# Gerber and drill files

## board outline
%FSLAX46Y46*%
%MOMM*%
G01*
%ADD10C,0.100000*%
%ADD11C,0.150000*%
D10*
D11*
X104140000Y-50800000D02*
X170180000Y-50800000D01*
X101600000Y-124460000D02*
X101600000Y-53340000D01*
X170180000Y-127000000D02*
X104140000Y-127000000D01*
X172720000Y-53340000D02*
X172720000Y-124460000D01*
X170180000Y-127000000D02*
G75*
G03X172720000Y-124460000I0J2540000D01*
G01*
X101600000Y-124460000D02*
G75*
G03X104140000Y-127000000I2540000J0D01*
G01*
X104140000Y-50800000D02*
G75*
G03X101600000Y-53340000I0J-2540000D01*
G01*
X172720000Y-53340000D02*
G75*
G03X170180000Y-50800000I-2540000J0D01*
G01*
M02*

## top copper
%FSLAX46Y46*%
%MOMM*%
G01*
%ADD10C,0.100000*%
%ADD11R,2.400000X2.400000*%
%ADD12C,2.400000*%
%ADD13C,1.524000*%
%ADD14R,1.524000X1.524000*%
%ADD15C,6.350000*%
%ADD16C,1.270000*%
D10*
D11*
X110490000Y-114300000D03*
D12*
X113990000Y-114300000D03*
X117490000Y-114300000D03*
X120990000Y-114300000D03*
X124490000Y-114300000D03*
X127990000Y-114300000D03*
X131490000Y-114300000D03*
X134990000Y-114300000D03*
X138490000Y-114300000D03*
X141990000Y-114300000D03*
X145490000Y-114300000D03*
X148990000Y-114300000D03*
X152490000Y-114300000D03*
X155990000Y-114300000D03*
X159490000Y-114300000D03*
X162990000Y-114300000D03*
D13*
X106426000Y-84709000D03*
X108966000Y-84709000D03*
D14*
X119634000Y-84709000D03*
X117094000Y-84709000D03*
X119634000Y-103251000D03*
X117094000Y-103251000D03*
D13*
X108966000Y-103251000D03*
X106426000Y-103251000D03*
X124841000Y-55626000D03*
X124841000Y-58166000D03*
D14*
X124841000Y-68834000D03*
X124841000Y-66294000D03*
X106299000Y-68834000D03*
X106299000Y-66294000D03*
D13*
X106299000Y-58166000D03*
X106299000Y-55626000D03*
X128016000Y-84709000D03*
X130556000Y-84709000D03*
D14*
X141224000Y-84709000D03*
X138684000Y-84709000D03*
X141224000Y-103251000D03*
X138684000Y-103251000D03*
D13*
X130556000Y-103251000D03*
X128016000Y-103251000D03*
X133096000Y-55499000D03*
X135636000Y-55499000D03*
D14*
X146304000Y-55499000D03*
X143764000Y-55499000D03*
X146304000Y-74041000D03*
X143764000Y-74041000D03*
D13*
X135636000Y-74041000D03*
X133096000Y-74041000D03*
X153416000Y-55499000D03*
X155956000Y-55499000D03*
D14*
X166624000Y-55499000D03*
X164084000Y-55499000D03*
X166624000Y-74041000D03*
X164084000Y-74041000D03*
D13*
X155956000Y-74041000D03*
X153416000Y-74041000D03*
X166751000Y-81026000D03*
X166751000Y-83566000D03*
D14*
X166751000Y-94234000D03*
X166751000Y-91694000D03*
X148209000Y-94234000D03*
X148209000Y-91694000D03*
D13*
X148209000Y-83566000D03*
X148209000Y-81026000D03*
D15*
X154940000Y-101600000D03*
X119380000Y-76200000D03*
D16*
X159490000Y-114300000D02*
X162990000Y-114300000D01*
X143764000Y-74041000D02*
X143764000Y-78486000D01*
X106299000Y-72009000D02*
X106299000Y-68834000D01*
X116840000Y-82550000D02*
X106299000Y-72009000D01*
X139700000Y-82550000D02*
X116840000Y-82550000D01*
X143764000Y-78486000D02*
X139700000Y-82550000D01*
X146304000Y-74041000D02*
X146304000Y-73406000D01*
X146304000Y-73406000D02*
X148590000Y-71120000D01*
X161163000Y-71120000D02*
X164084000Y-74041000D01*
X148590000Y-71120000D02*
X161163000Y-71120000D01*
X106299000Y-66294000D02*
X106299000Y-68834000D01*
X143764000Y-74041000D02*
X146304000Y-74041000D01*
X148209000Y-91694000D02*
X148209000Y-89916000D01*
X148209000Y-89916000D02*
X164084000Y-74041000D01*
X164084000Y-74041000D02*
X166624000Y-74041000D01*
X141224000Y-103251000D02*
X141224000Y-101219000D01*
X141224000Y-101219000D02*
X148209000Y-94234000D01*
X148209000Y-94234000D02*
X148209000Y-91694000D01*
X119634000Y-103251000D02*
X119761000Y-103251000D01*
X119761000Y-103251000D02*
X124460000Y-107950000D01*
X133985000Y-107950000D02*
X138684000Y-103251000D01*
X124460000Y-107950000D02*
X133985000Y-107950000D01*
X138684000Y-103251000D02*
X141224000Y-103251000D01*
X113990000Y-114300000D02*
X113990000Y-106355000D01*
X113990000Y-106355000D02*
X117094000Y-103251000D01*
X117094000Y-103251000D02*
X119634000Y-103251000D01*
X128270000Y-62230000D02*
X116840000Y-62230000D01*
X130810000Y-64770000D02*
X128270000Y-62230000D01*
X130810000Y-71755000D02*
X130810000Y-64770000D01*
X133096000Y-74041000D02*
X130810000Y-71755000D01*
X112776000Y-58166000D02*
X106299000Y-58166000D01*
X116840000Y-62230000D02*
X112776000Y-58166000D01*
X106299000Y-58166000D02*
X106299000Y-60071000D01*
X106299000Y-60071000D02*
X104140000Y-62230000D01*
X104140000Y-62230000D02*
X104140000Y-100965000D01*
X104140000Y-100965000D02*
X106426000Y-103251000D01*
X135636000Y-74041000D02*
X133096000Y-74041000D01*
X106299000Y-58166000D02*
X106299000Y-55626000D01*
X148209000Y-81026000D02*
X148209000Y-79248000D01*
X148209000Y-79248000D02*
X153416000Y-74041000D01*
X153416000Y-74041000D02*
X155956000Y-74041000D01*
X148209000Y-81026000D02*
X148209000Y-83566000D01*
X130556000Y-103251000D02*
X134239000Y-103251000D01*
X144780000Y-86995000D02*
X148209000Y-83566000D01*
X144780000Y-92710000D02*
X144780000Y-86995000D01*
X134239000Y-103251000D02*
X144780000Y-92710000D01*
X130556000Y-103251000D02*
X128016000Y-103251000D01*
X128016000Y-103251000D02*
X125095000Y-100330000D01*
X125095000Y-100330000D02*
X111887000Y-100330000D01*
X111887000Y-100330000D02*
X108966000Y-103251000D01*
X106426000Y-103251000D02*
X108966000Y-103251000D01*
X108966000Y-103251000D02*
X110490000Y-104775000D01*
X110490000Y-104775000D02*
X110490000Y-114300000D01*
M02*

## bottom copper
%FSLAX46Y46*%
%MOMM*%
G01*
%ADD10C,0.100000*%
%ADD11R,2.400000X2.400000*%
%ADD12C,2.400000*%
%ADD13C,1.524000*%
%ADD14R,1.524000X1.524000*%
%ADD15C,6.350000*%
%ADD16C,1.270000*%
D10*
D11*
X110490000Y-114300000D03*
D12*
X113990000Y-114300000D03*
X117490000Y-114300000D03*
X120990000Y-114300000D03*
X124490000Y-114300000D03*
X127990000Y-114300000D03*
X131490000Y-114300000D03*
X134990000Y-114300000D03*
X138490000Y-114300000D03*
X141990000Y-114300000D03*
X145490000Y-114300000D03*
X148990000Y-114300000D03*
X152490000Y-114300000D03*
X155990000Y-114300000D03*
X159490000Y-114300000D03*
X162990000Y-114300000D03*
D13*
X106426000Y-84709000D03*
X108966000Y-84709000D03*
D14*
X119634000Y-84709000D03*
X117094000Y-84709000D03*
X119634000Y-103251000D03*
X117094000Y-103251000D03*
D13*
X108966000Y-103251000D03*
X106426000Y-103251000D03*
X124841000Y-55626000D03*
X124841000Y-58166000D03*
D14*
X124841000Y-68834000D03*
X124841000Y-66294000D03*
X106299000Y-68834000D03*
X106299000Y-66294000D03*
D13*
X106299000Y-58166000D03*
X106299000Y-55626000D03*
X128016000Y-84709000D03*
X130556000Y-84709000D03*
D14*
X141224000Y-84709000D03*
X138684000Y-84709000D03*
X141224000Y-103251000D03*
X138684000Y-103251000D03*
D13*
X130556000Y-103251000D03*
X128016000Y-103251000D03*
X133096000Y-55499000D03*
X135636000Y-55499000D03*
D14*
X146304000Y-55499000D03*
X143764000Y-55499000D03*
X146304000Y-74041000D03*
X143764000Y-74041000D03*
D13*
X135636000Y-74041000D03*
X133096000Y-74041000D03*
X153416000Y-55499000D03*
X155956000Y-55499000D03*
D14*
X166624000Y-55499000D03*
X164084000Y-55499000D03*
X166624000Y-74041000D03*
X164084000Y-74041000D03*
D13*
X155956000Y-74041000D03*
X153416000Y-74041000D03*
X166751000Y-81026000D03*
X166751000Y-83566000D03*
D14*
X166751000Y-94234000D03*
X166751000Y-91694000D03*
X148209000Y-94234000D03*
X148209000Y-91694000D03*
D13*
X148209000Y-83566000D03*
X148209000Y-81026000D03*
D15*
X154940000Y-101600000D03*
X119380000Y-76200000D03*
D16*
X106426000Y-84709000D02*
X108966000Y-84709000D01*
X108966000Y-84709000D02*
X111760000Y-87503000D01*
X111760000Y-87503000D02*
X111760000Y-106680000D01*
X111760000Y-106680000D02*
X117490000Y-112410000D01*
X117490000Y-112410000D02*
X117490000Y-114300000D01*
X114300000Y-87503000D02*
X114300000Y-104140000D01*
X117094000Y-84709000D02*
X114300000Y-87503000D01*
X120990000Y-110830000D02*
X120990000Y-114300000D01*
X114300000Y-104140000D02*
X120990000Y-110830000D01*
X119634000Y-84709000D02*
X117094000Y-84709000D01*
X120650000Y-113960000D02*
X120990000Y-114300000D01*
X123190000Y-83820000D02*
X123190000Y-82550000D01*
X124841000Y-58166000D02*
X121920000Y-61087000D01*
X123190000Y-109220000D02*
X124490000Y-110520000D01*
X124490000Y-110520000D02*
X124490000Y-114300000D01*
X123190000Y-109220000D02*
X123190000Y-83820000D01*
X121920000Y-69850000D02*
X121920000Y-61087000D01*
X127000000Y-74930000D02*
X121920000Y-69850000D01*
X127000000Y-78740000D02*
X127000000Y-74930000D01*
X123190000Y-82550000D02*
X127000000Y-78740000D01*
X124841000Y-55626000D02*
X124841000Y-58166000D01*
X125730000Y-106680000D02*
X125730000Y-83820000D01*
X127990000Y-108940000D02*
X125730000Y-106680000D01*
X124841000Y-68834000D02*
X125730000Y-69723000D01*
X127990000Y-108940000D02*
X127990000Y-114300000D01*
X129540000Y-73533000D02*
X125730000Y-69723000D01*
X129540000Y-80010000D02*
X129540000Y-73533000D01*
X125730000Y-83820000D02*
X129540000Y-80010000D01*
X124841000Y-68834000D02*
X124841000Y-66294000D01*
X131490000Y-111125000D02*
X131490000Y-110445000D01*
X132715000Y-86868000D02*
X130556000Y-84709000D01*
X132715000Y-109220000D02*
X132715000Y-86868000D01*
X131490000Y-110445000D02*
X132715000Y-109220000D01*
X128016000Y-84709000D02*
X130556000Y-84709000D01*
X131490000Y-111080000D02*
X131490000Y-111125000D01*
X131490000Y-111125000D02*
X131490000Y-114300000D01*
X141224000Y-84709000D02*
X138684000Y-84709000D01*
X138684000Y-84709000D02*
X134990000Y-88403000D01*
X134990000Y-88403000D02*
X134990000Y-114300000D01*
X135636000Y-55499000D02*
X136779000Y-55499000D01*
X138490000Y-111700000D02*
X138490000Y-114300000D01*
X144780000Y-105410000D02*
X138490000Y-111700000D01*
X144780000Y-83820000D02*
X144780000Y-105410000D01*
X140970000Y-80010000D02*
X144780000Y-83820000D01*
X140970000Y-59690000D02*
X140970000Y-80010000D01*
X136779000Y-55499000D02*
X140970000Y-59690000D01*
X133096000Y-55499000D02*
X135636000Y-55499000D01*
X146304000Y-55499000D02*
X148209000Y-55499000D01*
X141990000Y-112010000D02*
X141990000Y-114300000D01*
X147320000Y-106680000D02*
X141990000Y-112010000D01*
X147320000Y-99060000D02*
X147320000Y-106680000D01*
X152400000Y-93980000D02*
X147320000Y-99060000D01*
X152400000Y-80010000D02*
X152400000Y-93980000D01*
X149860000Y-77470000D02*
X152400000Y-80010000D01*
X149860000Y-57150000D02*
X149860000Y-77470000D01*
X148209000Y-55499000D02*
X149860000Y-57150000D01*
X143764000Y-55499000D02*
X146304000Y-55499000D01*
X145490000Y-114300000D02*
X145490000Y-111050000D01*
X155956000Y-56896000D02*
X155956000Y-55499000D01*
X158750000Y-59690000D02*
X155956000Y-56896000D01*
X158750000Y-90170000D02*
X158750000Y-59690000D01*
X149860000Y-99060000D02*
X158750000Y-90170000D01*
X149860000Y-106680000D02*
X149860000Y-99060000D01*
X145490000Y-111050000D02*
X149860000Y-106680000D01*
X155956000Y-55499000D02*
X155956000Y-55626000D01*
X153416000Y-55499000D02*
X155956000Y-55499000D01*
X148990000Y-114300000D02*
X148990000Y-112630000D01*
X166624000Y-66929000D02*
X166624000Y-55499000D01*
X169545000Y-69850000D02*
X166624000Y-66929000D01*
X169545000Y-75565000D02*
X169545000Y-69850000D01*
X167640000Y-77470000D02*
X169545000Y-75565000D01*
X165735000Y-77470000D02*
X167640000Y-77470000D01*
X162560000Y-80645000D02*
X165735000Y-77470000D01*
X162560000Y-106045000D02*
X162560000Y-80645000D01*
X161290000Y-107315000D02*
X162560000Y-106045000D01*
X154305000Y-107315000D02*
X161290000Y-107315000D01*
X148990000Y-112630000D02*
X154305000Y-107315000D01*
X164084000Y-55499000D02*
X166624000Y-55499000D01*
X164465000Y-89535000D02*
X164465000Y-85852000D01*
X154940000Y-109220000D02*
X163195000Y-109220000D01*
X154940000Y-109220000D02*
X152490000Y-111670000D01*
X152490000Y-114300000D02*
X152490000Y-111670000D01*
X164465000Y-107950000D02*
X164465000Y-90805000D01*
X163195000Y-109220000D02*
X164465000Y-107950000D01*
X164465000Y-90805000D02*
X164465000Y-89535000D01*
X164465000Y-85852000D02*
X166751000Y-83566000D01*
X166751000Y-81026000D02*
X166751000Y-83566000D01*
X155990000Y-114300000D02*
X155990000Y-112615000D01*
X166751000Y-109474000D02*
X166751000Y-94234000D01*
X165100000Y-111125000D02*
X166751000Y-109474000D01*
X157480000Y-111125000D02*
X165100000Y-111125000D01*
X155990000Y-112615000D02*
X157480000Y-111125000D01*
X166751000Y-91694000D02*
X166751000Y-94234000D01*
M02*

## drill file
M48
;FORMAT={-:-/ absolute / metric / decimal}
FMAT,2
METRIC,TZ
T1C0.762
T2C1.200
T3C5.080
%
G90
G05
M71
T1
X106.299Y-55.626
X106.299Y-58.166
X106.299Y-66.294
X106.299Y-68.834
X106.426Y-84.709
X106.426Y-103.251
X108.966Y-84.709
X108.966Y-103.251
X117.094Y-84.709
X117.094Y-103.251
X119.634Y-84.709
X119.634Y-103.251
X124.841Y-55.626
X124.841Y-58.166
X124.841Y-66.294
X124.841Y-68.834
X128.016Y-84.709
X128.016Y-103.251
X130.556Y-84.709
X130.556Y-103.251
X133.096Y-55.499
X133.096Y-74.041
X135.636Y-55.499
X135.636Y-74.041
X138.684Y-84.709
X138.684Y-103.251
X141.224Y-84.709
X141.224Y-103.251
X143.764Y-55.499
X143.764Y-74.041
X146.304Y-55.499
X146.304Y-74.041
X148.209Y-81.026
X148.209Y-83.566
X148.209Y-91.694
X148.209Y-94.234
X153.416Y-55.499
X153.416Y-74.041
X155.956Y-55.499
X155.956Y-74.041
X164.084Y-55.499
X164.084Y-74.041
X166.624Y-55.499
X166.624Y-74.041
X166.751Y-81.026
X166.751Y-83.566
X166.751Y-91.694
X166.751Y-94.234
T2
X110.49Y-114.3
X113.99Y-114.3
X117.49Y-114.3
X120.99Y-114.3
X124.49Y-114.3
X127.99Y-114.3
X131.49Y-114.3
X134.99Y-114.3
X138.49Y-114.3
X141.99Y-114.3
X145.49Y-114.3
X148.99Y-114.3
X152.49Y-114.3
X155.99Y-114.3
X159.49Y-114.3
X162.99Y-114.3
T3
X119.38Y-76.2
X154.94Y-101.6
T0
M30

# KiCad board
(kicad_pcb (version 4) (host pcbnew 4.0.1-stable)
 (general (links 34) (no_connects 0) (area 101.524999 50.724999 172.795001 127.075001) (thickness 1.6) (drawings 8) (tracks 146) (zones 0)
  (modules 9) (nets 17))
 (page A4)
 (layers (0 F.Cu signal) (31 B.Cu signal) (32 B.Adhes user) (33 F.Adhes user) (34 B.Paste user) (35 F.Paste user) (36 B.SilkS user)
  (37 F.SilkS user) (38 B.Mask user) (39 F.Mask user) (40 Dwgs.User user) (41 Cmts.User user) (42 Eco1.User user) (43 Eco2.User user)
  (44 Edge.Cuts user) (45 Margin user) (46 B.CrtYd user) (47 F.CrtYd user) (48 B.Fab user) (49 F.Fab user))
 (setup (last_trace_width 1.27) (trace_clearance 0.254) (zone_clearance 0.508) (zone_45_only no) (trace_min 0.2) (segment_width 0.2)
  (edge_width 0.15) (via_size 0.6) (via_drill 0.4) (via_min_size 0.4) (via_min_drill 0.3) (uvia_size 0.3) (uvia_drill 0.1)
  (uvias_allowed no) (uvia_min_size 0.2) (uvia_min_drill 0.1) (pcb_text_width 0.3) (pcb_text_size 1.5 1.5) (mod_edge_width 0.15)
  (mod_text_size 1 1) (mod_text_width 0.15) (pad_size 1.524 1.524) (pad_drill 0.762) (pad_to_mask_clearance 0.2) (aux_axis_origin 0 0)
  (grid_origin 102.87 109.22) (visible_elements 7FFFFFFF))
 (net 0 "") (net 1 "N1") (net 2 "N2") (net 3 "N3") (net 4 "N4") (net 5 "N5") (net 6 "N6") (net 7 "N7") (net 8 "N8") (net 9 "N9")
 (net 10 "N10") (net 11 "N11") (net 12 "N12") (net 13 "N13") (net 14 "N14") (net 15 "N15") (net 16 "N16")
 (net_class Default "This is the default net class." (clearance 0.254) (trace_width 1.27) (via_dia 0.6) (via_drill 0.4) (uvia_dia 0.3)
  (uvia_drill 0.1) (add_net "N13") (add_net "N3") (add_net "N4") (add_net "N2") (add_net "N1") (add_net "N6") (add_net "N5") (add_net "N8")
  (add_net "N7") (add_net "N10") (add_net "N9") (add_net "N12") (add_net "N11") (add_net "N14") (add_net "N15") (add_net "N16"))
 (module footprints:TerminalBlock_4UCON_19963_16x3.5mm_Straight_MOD (layer F.Cu) (at 110.49 114.3)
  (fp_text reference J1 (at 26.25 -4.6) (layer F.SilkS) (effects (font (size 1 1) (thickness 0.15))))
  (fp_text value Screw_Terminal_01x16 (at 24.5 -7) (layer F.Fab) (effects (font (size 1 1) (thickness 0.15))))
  (pad 1 thru_hole rect (at 0 0) (size 2.4 2.4) (drill 1.2) (layers *.Cu *.Mask))
  (pad 2 thru_hole circle (at 3.5 0) (size 2.4 2.4) (drill 1.2) (layers *.Cu *.Mask))
  (pad 3 thru_hole circle (at 7 0) (size 2.4 2.4) (drill 1.2) (layers *.Cu *.Mask))
  (pad 4 thru_hole circle (at 10.5 0) (size 2.4 2.4) (drill 1.2) (layers *.Cu *.Mask))
  (pad 5 thru_hole circle (at 14 0) (size 2.4 2.4) (drill 1.2) (layers *.Cu *.Mask))
  (pad 6 thru_hole circle (at 17.5 0) (size 2.4 2.4) (drill 1.2) (layers *.Cu *.Mask))
  (pad 7 thru_hole circle (at 21 0) (size 2.4 2.4) (drill 1.2) (layers *.Cu *.Mask))
  (pad 8 thru_hole circle (at 24.5 0) (size 2.4 2.4) (drill 1.2) (layers *.Cu *.Mask))
  (pad 9 thru_hole circle (at 28 0) (size 2.4 2.4) (drill 1.2) (layers *.Cu *.Mask))
  (pad 10 thru_hole circle (at 31.5 0) (size 2.4 2.4) (drill 1.2) (layers *.Cu *.Mask))
  (pad 11 thru_hole circle (at 35 0) (size 2.4 2.4) (drill 1.2) (layers *.Cu *.Mask))
  (pad 12 thru_hole circle (at 38.5 0) (size 2.4 2.4) (drill 1.2) (layers *.Cu *.Mask))
  (pad 13 thru_hole circle (at 42 0) (size 2.4 2.4) (drill 1.2) (layers *.Cu *.Mask))
  (pad 14 thru_hole circle (at 45.5 0) (size 2.4 2.4) (drill 1.2) (layers *.Cu *.Mask))
  (pad 15 thru_hole circle (at 49 0) (size 2.4 2.4) (drill 1.2) (layers *.Cu *.Mask))
  (pad 16 thru_hole circle (at 52.5 0) (size 2.4 2.4) (drill 1.2) (layers *.Cu *.Mask)))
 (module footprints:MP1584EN (layer F.Cu) (at 113.03 93.98 90)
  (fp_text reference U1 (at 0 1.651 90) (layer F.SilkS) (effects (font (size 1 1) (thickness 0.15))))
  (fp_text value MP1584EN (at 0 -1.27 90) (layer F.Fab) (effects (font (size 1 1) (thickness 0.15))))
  (pad 4 thru_hole circle (at 9.271 -6.604 90) (size 1.524 1.524) (drill 0.762) (layers *.Cu *.Mask) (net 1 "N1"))
  (pad 4 thru_hole circle (at 9.271 -4.064 90) (size 1.524 1.524) (drill 0.762) (layers *.Cu *.Mask) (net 1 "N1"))
  (pad 3 thru_hole rect (at 9.271 6.604 90) (size 1.524 1.524) (drill 0.762) (layers *.Cu *.Mask) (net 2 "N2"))
  (pad 3 thru_hole rect (at 9.271 4.064 90) (size 1.524 1.524) (drill 0.762) (layers *.Cu *.Mask) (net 2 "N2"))
  (pad 1 thru_hole rect (at -9.271 6.604 90) (size 1.524 1.524) (drill 0.762) (layers *.Cu *.Mask) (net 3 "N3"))
  (pad 1 thru_hole rect (at -9.271 4.064 90) (size 1.524 1.524) (drill 0.762) (layers *.Cu *.Mask) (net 3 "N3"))
  (pad 2 thru_hole circle (at -9.271 -4.064 90) (size 1.524 1.524) (drill 0.762) (layers *.Cu *.Mask) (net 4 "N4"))
  (pad 2 thru_hole circle (at -9.271 -6.604 90) (size 1.524 1.524) (drill 0.762) (layers *.Cu *.Mask) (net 4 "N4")))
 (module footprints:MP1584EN (layer F.Cu) (at 115.57 62.23)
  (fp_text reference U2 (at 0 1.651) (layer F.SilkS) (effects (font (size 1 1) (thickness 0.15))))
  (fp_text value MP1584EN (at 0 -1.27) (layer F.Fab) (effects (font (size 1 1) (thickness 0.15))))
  (pad 4 thru_hole circle (at 9.271 -6.604) (size 1.524 1.524) (drill 0.762) (layers *.Cu *.Mask) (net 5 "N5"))
  (pad 4 thru_hole circle (at 9.271 -4.064) (size 1.524 1.524) (drill 0.762) (layers *.Cu *.Mask) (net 5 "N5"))
  (pad 3 thru_hole rect (at 9.271 6.604) (size 1.524 1.524) (drill 0.762) (layers *.Cu *.Mask) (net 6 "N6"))
  (pad 3 thru_hole rect (at 9.271 4.064) (size 1.524 1.524) (drill 0.762) (layers *.Cu *.Mask) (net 6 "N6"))
  (pad 1 thru_hole rect (at -9.271 6.604) (size 1.524 1.524) (drill 0.762) (layers *.Cu *.Mask) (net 3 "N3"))
  (pad 1 thru_hole rect (at -9.271 4.064) (size 1.524 1.524) (drill 0.762) (layers *.Cu *.Mask) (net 3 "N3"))
  (pad 2 thru_hole circle (at -9.271 -4.064) (size 1.524 1.524) (drill 0.762) (layers *.Cu *.Mask) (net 4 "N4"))
  (pad 2 thru_hole circle (at -9.271 -6.604) (size 1.524 1.524) (drill 0.762) (layers *.Cu *.Mask) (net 4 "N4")))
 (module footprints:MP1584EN (layer F.Cu) (at 134.62 93.98 90)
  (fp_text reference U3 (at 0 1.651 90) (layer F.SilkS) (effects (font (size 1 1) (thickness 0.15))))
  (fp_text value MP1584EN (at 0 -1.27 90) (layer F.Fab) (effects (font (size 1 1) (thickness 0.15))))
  (pad 4 thru_hole circle (at 9.271 -6.604 90) (size 1.524 1.524) (drill 0.762) (layers *.Cu *.Mask) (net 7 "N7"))
  (pad 4 thru_hole circle (at 9.271 -4.064 90) (size 1.524 1.524) (drill 0.762) (layers *.Cu *.Mask) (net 7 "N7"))
  (pad 3 thru_hole rect (at 9.271 6.604 90) (size 1.524 1.524) (drill 0.762) (layers *.Cu *.Mask) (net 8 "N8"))
  (pad 3 thru_hole rect (at 9.271 4.064 90) (size 1.524 1.524) (drill 0.762) (layers *.Cu *.Mask) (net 8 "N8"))
  (pad 1 thru_hole rect (at -9.271 6.604 90) (size 1.524 1.524) (drill 0.762) (layers *.Cu *.Mask) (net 3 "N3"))
  (pad 1 thru_hole rect (at -9.271 4.064 90) (size 1.524 1.524) (drill 0.762) (layers *.Cu *.Mask) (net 3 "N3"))
  (pad 2 thru_hole circle (at -9.271 -4.064 90) (size 1.524 1.524) (drill 0.762) (layers *.Cu *.Mask) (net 4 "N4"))
  (pad 2 thru_hole circle (at -9.271 -6.604 90) (size 1.524 1.524) (drill 0.762) (layers *.Cu *.Mask) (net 4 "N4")))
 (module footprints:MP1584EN (layer F.Cu) (at 139.7 64.77 90)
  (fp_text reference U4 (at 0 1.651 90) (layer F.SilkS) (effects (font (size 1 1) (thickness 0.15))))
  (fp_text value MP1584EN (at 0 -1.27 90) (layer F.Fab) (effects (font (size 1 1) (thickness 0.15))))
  (pad 4 thru_hole circle (at 9.271 -6.604 90) (size 1.524 1.524) (drill 0.762) (layers *.Cu *.Mask) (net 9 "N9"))
  (pad 4 thru_hole circle (at 9.271 -4.064 90) (size 1.524 1.524) (drill 0.762) (layers *.Cu *.Mask) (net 9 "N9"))
  (pad 3 thru_hole rect (at 9.271 6.604 90) (size 1.524 1.524) (drill 0.762) (layers *.Cu *.Mask) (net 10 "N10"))
  (pad 3 thru_hole rect (at 9.271 4.064 90) (size 1.524 1.524) (drill 0.762) (layers *.Cu *.Mask) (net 10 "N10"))
  (pad 1 thru_hole rect (at -9.271 6.604 90) (size 1.524 1.524) (drill 0.762) (layers *.Cu *.Mask) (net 3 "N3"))
  (pad 1 thru_hole rect (at -9.271 4.064 90) (size 1.524 1.524) (drill 0.762) (layers *.Cu *.Mask) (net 3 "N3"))
  (pad 2 thru_hole circle (at -9.271 -4.064 90) (size 1.524 1.524) (drill 0.762) (layers *.Cu *.Mask) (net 4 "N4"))
  (pad 2 thru_hole circle (at -9.271 -6.604 90) (size 1.524 1.524) (drill 0.762) (layers *.Cu *.Mask) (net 4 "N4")))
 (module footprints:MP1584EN (layer F.Cu) (at 160.02 64.77 90)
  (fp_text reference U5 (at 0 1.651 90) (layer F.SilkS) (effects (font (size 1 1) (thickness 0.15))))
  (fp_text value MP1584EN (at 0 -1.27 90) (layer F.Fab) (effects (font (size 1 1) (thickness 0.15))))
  (pad 4 thru_hole circle (at 9.271 -6.604 90) (size 1.524 1.524) (drill 0.762) (layers *.Cu *.Mask) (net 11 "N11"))
  (pad 4 thru_hole circle (at 9.271 -4.064 90) (size 1.524 1.524) (drill 0.762) (layers *.Cu *.Mask) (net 11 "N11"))
  (pad 3 thru_hole rect (at 9.271 6.604 90) (size 1.524 1.524) (drill 0.762) (layers *.Cu *.Mask) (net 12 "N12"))
  (pad 3 thru_hole rect (at 9.271 4.064 90) (size 1.524 1.524) (drill 0.762) (layers *.Cu *.Mask) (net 12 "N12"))
  (pad 1 thru_hole rect (at -9.271 6.604 90) (size 1.524 1.524) (drill 0.762) (layers *.Cu *.Mask) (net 3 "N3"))
  (pad 1 thru_hole rect (at -9.271 4.064 90) (size 1.524 1.524) (drill 0.762) (layers *.Cu *.Mask) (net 3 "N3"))
  (pad 2 thru_hole circle (at -9.271 -4.064 90) (size 1.524 1.524) (drill 0.762) (layers *.Cu *.Mask) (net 4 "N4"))
  (pad 2 thru_hole circle (at -9.271 -6.604 90) (size 1.524 1.524) (drill 0.762) (layers *.Cu *.Mask) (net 4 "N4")))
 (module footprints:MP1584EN (layer F.Cu) (at 157.48 87.63)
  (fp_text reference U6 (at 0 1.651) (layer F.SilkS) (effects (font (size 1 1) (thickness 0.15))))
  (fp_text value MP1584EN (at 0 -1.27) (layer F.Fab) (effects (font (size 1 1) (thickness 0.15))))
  (pad 4 thru_hole circle (at 9.271 -6.604) (size 1.524 1.524) (drill 0.762) (layers *.Cu *.Mask) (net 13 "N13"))
  (pad 4 thru_hole circle (at 9.271 -4.064) (size 1.524 1.524) (drill 0.762) (layers *.Cu *.Mask) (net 13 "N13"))
  (pad 3 thru_hole rect (at 9.271 6.604) (size 1.524 1.524) (drill 0.762) (layers *.Cu *.Mask) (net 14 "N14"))
  (pad 3 thru_hole rect (at 9.271 4.064) (size 1.524 1.524) (drill 0.762) (layers *.Cu *.Mask) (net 14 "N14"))
  (pad 1 thru_hole rect (at -9.271 6.604) (size 1.524 1.524) (drill 0.762) (layers *.Cu *.Mask) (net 3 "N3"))
  (pad 1 thru_hole rect (at -9.271 4.064) (size 1.524 1.524) (drill 0.762) (layers *.Cu *.Mask) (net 3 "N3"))
  (pad 2 thru_hole circle (at -9.271 -4.064) (size 1.524 1.524) (drill 0.762) (layers *.Cu *.Mask) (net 4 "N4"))
  (pad 2 thru_hole circle (at -9.271 -6.604) (size 1.524 1.524) (drill 0.762) (layers *.Cu *.Mask) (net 4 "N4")))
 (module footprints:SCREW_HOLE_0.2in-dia (layer F.Cu) (at 154.94 101.6)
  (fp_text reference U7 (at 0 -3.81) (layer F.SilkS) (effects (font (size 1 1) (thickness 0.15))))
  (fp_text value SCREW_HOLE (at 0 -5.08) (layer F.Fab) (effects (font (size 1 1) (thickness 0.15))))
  (pad 1 thru_hole circle (at 0 0) (size 6.35 6.35) (drill 5.08) (layers *.Cu *.Mask) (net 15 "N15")))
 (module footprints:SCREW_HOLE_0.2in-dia (layer F.Cu) (at 119.38 76.2)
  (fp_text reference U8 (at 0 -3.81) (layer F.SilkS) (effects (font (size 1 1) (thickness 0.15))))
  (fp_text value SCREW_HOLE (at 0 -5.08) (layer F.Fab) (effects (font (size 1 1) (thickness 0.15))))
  (pad 1 thru_hole circle (at 0 0) (size 6.35 6.35) (drill 5.08) (layers *.Cu *.Mask) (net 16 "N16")))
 (gr_line (start 104.14 50.8) (end 170.18 50.8) (angle 90) (layer Edge.Cuts) (width 0.15))
 (gr_line (start 101.6 124.46) (end 101.6 53.34) (angle 90) (layer Edge.Cuts) (width 0.15))
 (gr_line (start 170.18 127) (end 104.14 127) (angle 90) (layer Edge.Cuts) (width 0.15))
 (gr_line (start 172.72 53.34) (end 172.72 124.46) (angle 90) (layer Edge.Cuts) (width 0.15))
 (gr_arc (start 170.18 124.46) (end 172.72 124.46) (angle 90) (layer Edge.Cuts) (width 0.15))
 (gr_arc (start 104.14 124.46) (end 104.14 127) (angle 90) (layer Edge.Cuts) (width 0.15))
 (gr_arc (start 104.14 53.34) (end 101.6 53.34) (angle 90) (layer Edge.Cuts) (width 0.15))
 (gr_arc (start 170.18 53.34) (end 170.18 50.8) (angle 90) (layer Edge.Cuts) (width 0.15))
 (segment (start 159.49 114.3) (end 162.99 114.3) (width 1.27) (layer F.Cu) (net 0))
 (segment (start 106.426 84.709) (end 108.966 84.709) (width 1.27) (layer B.Cu) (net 1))
 (segment (start 108.966 84.709) (end 111.76 87.503) (width 1.27) (layer B.Cu) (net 1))
 (segment (start 111.76 87.503) (end 111.76 106.68) (width 1.27) (layer B.Cu) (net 1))
 (segment (start 111.76 106.68) (end 117.49 112.41) (width 1.27) (layer B.Cu) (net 1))
 (segment (start 117.49 112.41) (end 117.49 114.3) (width 1.27) (layer B.Cu) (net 1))
 (segment (start 114.3 87.503) (end 114.3 104.14) (width 1.27) (layer B.Cu) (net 2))
 (segment (start 117.094 84.709) (end 114.3 87.503) (width 1.27) (layer B.Cu) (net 2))
 (segment (start 120.99 110.83) (end 120.99 114.3) (width 1.27) (layer B.Cu) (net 2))
 (segment (start 114.3 104.14) (end 120.99 110.83) (width 1.27) (layer B.Cu) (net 2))
 (segment (start 119.634 84.709) (end 117.094 84.709) (width 1.27) (layer B.Cu) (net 2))
 (segment (start 120.65 113.96) (end 120.99 114.3) (width 1.27) (layer B.Cu) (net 2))
 (segment (start 143.764 74.041) (end 143.764 78.486) (width 1.27) (layer F.Cu) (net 3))
 (segment (start 106.299 72.009) (end 106.299 68.834) (width 1.27) (layer F.Cu) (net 3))
 (segment (start 116.84 82.55) (end 106.299 72.009) (width 1.27) (layer F.Cu) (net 3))
 (segment (start 139.7 82.55) (end 116.84 82.55) (width 1.27) (layer F.Cu) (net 3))
 (segment (start 143.764 78.486) (end 139.7 82.55) (width 1.27) (layer F.Cu) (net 3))
 (segment (start 146.304 74.041) (end 146.304 73.406) (width 1.27) (layer F.Cu) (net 3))
 (segment (start 146.304 73.406) (end 148.59 71.12) (width 1.27) (layer F.Cu) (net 3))
 (segment (start 161.163 71.12) (end 164.084 74.041) (width 1.27) (layer F.Cu) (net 3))
 (segment (start 148.59 71.12) (end 161.163 71.12) (width 1.27) (layer F.Cu) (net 3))
 (segment (start 106.299 66.294) (end 106.299 68.834) (width 1.27) (layer F.Cu) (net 3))
 (segment (start 143.764 74.041) (end 146.304 74.041) (width 1.27) (layer F.Cu) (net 3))
 (segment (start 148.209 91.694) (end 148.209 89.916) (width 1.27) (layer F.Cu) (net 3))
 (segment (start 148.209 89.916) (end 164.084 74.041) (width 1.27) (layer F.Cu) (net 3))
 (segment (start 164.084 74.041) (end 166.624 74.041) (width 1.27) (layer F.Cu) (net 3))
 (segment (start 141.224 103.251) (end 141.224 101.219) (width 1.27) (layer F.Cu) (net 3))
 (segment (start 141.224 101.219) (end 148.209 94.234) (width 1.27) (layer F.Cu) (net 3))
 (segment (start 148.209 94.234) (end 148.209 91.694) (width 1.27) (layer F.Cu) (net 3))
 (segment (start 119.634 103.251) (end 119.761 103.251) (width 1.27) (layer F.Cu) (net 3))
 (segment (start 119.761 103.251) (end 124.46 107.95) (width 1.27) (layer F.Cu) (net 3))
 (segment (start 133.985 107.95) (end 138.684 103.251) (width 1.27) (layer F.Cu) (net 3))
 (segment (start 124.46 107.95) (end 133.985 107.95) (width 1.27) (layer F.Cu) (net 3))
 (segment (start 138.684 103.251) (end 141.224 103.251) (width 1.27) (layer F.Cu) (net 3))
 (segment (start 113.99 114.3) (end 113.99 106.355) (width 1.27) (layer F.Cu) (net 3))
 (segment (start 113.99 106.355) (end 117.094 103.251) (width 1.27) (layer F.Cu) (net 3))
 (segment (start 117.094 103.251) (end 119.634 103.251) (width 1.27) (layer F.Cu) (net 3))
 (segment (start 128.27 62.23) (end 116.84 62.23) (width 1.27) (layer F.Cu) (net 4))
 (segment (start 130.81 64.77) (end 128.27 62.23) (width 1.27) (layer F.Cu) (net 4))
 (segment (start 130.81 71.755) (end 130.81 64.77) (width 1.27) (layer F.Cu) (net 4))
 (segment (start 133.096 74.041) (end 130.81 71.755) (width 1.27) (layer F.Cu) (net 4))
 (segment (start 112.776 58.166) (end 106.299 58.166) (width 1.27) (layer F.Cu) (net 4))
 (segment (start 116.84 62.23) (end 112.776 58.166) (width 1.27) (layer F.Cu) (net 4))
 (segment (start 106.299 58.166) (end 106.299 60.071) (width 1.27) (layer F.Cu) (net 4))
 (segment (start 106.299 60.071) (end 104.14 62.23) (width 1.27) (layer F.Cu) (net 4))
 (segment (start 104.14 62.23) (end 104.14 100.965) (width 1.27) (layer F.Cu) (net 4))
 (segment (start 104.14 100.965) (end 106.426 103.251) (width 1.27) (layer F.Cu) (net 4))
 (segment (start 135.636 74.041) (end 133.096 74.041) (width 1.27) (layer F.Cu) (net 4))
 (segment (start 106.299 58.166) (end 106.299 55.626) (width 1.27) (layer F.Cu) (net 4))
 (segment (start 148.209 81.026) (end 148.209 79.248) (width 1.27) (layer F.Cu) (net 4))
 (segment (start 148.209 79.248) (end 153.416 74.041) (width 1.27) (layer F.Cu) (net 4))
 (segment (start 153.416 74.041) (end 155.956 74.041) (width 1.27) (layer F.Cu) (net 4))
 (segment (start 148.209 81.026) (end 148.209 83.566) (width 1.27) (layer F.Cu) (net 4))
 (segment (start 130.556 103.251) (end 134.239 103.251) (width 1.27) (layer F.Cu) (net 4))
 (segment (start 144.78 86.995) (end 148.209 83.566) (width 1.27) (layer F.Cu) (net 4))
 (segment (start 144.78 92.71) (end 144.78 86.995) (width 1.27) (layer F.Cu) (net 4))
 (segment (start 134.239 103.251) (end 144.78 92.71) (width 1.27) (layer F.Cu) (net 4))
 (segment (start 130.556 103.251) (end 128.016 103.251) (width 1.27) (layer F.Cu) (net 4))
 (segment (start 128.016 103.251) (end 125.095 100.33) (width 1.27) (layer F.Cu) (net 4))
 (segment (start 125.095 100.33) (end 111.887 100.33) (width 1.27) (layer F.Cu) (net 4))
 (segment (start 111.887 100.33) (end 108.966 103.251) (width 1.27) (layer F.Cu) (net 4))
 (segment (start 106.426 103.251) (end 108.966 103.251) (width 1.27) (layer F.Cu) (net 4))
 (segment (start 108.966 103.251) (end 110.49 104.775) (width 1.27) (layer F.Cu) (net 4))
 (segment (start 110.49 104.775) (end 110.49 114.3) (width 1.27) (layer F.Cu) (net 4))
 (segment (start 123.19 83.82) (end 123.19 82.55) (width 1.27) (layer B.Cu) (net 5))
 (segment (start 124.841 58.166) (end 121.92 61.087) (width 1.27) (layer B.Cu) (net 5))
 (segment (start 123.19 109.22) (end 124.49 110.52) (width 1.27) (layer B.Cu) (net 5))
 (segment (start 124.49 110.52) (end 124.49 114.3) (width 1.27) (layer B.Cu) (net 5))
 (segment (start 123.19 109.22) (end 123.19 83.82) (width 1.27) (layer B.Cu) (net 5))
 (segment (start 121.92 69.85) (end 121.92 61.087) (width 1.27) (layer B.Cu) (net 5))
 (segment (start 127 74.93) (end 121.92 69.85) (width 1.27) (layer B.Cu) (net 5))
 (segment (start 127 78.74) (end 127 74.93) (width 1.27) (layer B.Cu) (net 5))
 (segment (start 123.19 82.55) (end 127 78.74) (width 1.27) (layer B.Cu) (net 5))
 (segment (start 124.841 55.626) (end 124.841 58.166) (width 1.27) (layer B.Cu) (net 5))
 (segment (start 125.73 106.68) (end 125.73 83.82) (width 1.27) (layer B.Cu) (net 6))
 (segment (start 127.99 108.94) (end 125.73 106.68) (width 1.27) (layer B.Cu) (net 6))
 (segment (start 124.841 68.834) (end 125.73 69.723) (width 1.27) (layer B.Cu) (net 6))
 (segment (start 127.99 108.94) (end 127.99 114.3) (width 1.27) (layer B.Cu) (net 6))
 (segment (start 129.54 73.533) (end 125.73 69.723) (width 1.27) (layer B.Cu) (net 6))
 (segment (start 129.54 80.01) (end 129.54 73.533) (width 1.27) (layer B.Cu) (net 6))
 (segment (start 125.73 83.82) (end 129.54 80.01) (width 1.27) (layer B.Cu) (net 6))
 (segment (start 124.841 68.834) (end 124.841 66.294) (width 1.27) (layer B.Cu) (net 6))
 (segment (start 131.49 111.125) (end 131.49 110.445) (width 1.27) (layer B.Cu) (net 7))
 (segment (start 132.715 86.868) (end 130.556 84.709) (width 1.27) (layer B.Cu) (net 7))
 (segment (start 132.715 109.22) (end 132.715 86.868) (width 1.27) (layer B.Cu) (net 7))
 (segment (start 131.49 110.445) (end 132.715 109.22) (width 1.27) (layer B.Cu) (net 7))
 (segment (start 128.016 84.709) (end 130.556 84.709) (width 1.27) (layer B.Cu) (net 7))
 (segment (start 131.49 111.08) (end 131.49 111.125) (width 1.27) (layer B.Cu) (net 7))
 (segment (start 131.49 111.125) (end 131.49 114.3) (width 1.27) (layer B.Cu) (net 7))
 (segment (start 141.224 84.709) (end 138.684 84.709) (width 1.27) (layer B.Cu) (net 8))
 (segment (start 138.684 84.709) (end 134.99 88.403) (width 1.27) (layer B.Cu) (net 8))
 (segment (start 134.99 88.403) (end 134.99 114.3) (width 1.27) (layer B.Cu) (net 8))
 (segment (start 135.636 55.499) (end 136.779 55.499) (width 1.27) (layer B.Cu) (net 9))
 (segment (start 138.49 111.7) (end 138.49 114.3) (width 1.27) (layer B.Cu) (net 9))
 (segment (start 144.78 105.41) (end 138.49 111.7) (width 1.27) (layer B.Cu) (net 9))
 (segment (start 144.78 83.82) (end 144.78 105.41) (width 1.27) (layer B.Cu) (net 9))
 (segment (start 140.97 80.01) (end 144.78 83.82) (width 1.27) (layer B.Cu) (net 9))
 (segment (start 140.97 59.69) (end 140.97 80.01) (width 1.27) (layer B.Cu) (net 9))
 (segment (start 136.779 55.499) (end 140.97 59.69) (width 1.27) (layer B.Cu) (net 9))
 (segment (start 133.096 55.499) (end 135.636 55.499) (width 1.27) (layer B.Cu) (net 9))
 (segment (start 146.304 55.499) (end 148.209 55.499) (width 1.27) (layer B.Cu) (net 10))
 (segment (start 141.99 112.01) (end 141.99 114.3) (width 1.27) (layer B.Cu) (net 10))
 (segment (start 147.32 106.68) (end 141.99 112.01) (width 1.27) (layer B.Cu) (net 10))
 (segment (start 147.32 99.06) (end 147.32 106.68) (width 1.27) (layer B.Cu) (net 10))
 (segment (start 152.4 93.98) (end 147.32 99.06) (width 1.27) (layer B.Cu) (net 10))
 (segment (start 152.4 80.01) (end 152.4 93.98) (width 1.27) (layer B.Cu) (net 10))
 (segment (start 149.86 77.47) (end 152.4 80.01) (width 1.27) (layer B.Cu) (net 10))
 (segment (start 149.86 57.15) (end 149.86 77.47) (width 1.27) (layer B.Cu) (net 10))
 (segment (start 148.209 55.499) (end 149.86 57.15) (width 1.27) (layer B.Cu) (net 10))
 (segment (start 143.764 55.499) (end 146.304 55.499) (width 1.27) (layer B.Cu) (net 10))
 (segment (start 145.49 114.3) (end 145.49 111.05) (width 1.27) (layer B.Cu) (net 11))
 (segment (start 155.956 56.896) (end 155.956 55.499) (width 1.27) (layer B.Cu) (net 11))
 (segment (start 158.75 59.69) (end 155.956 56.896) (width 1.27) (layer B.Cu) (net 11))
 (segment (start 158.75 90.17) (end 158.75 59.69) (width 1.27) (layer B.Cu) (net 11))
 (segment (start 149.86 99.06) (end 158.75 90.17) (width 1.27) (layer B.Cu) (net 11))
 (segment (start 149.86 106.68) (end 149.86 99.06) (width 1.27) (layer B.Cu) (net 11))
 (segment (start 145.49 111.05) (end 149.86 106.68) (width 1.27) (layer B.Cu) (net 11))
 (segment (start 155.956 55.499) (end 155.956 55.626) (width 1.27) (layer B.Cu) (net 11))
 (segment (start 153.416 55.499) (end 155.956 55.499) (width 1.27) (layer B.Cu) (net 11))
 (segment (start 148.99 114.3) (end 148.99 112.63) (width 1.27) (layer B.Cu) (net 12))
 (segment (start 166.624 66.929) (end 166.624 55.499) (width 1.27) (layer B.Cu) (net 12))
 (segment (start 169.545 69.85) (end 166.624 66.929) (width 1.27) (layer B.Cu) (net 12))
 (segment (start 169.545 75.565) (end 169.545 69.85) (width 1.27) (layer B.Cu) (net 12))
 (segment (start 167.64 77.47) (end 169.545 75.565) (width 1.27) (layer B.Cu) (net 12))
 (segment (start 165.735 77.47) (end 167.64 77.47) (width 1.27) (layer B.Cu) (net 12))
 (segment (start 162.56 80.645) (end 165.735 77.47) (width 1.27) (layer B.Cu) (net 12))
 (segment (start 162.56 106.045) (end 162.56 80.645) (width 1.27) (layer B.Cu) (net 12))
 (segment (start 161.29 107.315) (end 162.56 106.045) (width 1.27) (layer B.Cu) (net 12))
 (segment (start 154.305 107.315) (end 161.29 107.315) (width 1.27) (layer B.Cu) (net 12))
 (segment (start 148.99 112.63) (end 154.305 107.315) (width 1.27) (layer B.Cu) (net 12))
 (segment (start 164.084 55.499) (end 166.624 55.499) (width 1.27) (layer B.Cu) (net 12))
 (segment (start 164.465 89.535) (end 164.465 85.852) (width 1.27) (layer B.Cu) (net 13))
 (segment (start 154.94 109.22) (end 163.195 109.22) (width 1.27) (layer B.Cu) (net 13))
 (segment (start 154.94 109.22) (end 152.49 111.67) (width 1.27) (layer B.Cu) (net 13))
 (segment (start 152.49 114.3) (end 152.49 111.67) (width 1.27) (layer B.Cu) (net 13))
 (segment (start 164.465 107.95) (end 164.465 90.805) (width 1.27) (layer B.Cu) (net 13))
 (segment (start 163.195 109.22) (end 164.465 107.95) (width 1.27) (layer B.Cu) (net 13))
 (segment (start 164.465 90.805) (end 164.465 89.535) (width 1.27) (layer B.Cu) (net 13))
 (segment (start 164.465 85.852) (end 166.751 83.566) (width 1.27) (layer B.Cu) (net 13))
 (segment (start 166.751 81.026) (end 166.751 83.566) (width 1.27) (layer B.Cu) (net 13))
 (segment (start 155.99 114.3) (end 155.99 112.615) (width 1.27) (layer B.Cu) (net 14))
 (segment (start 166.751 109.474) (end 166.751 94.234) (width 1.27) (layer B.Cu) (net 14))
 (segment (start 165.1 111.125) (end 166.751 109.474) (width 1.27) (layer B.Cu) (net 14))
 (segment (start 157.48 111.125) (end 165.1 111.125) (width 1.27) (layer B.Cu) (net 14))
 (segment (start 155.99 112.615) (end 157.48 111.125) (width 1.27) (layer B.Cu) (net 14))
 (segment (start 166.751 91.694) (end 166.751 94.234) (width 1.27) (layer B.Cu) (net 14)))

